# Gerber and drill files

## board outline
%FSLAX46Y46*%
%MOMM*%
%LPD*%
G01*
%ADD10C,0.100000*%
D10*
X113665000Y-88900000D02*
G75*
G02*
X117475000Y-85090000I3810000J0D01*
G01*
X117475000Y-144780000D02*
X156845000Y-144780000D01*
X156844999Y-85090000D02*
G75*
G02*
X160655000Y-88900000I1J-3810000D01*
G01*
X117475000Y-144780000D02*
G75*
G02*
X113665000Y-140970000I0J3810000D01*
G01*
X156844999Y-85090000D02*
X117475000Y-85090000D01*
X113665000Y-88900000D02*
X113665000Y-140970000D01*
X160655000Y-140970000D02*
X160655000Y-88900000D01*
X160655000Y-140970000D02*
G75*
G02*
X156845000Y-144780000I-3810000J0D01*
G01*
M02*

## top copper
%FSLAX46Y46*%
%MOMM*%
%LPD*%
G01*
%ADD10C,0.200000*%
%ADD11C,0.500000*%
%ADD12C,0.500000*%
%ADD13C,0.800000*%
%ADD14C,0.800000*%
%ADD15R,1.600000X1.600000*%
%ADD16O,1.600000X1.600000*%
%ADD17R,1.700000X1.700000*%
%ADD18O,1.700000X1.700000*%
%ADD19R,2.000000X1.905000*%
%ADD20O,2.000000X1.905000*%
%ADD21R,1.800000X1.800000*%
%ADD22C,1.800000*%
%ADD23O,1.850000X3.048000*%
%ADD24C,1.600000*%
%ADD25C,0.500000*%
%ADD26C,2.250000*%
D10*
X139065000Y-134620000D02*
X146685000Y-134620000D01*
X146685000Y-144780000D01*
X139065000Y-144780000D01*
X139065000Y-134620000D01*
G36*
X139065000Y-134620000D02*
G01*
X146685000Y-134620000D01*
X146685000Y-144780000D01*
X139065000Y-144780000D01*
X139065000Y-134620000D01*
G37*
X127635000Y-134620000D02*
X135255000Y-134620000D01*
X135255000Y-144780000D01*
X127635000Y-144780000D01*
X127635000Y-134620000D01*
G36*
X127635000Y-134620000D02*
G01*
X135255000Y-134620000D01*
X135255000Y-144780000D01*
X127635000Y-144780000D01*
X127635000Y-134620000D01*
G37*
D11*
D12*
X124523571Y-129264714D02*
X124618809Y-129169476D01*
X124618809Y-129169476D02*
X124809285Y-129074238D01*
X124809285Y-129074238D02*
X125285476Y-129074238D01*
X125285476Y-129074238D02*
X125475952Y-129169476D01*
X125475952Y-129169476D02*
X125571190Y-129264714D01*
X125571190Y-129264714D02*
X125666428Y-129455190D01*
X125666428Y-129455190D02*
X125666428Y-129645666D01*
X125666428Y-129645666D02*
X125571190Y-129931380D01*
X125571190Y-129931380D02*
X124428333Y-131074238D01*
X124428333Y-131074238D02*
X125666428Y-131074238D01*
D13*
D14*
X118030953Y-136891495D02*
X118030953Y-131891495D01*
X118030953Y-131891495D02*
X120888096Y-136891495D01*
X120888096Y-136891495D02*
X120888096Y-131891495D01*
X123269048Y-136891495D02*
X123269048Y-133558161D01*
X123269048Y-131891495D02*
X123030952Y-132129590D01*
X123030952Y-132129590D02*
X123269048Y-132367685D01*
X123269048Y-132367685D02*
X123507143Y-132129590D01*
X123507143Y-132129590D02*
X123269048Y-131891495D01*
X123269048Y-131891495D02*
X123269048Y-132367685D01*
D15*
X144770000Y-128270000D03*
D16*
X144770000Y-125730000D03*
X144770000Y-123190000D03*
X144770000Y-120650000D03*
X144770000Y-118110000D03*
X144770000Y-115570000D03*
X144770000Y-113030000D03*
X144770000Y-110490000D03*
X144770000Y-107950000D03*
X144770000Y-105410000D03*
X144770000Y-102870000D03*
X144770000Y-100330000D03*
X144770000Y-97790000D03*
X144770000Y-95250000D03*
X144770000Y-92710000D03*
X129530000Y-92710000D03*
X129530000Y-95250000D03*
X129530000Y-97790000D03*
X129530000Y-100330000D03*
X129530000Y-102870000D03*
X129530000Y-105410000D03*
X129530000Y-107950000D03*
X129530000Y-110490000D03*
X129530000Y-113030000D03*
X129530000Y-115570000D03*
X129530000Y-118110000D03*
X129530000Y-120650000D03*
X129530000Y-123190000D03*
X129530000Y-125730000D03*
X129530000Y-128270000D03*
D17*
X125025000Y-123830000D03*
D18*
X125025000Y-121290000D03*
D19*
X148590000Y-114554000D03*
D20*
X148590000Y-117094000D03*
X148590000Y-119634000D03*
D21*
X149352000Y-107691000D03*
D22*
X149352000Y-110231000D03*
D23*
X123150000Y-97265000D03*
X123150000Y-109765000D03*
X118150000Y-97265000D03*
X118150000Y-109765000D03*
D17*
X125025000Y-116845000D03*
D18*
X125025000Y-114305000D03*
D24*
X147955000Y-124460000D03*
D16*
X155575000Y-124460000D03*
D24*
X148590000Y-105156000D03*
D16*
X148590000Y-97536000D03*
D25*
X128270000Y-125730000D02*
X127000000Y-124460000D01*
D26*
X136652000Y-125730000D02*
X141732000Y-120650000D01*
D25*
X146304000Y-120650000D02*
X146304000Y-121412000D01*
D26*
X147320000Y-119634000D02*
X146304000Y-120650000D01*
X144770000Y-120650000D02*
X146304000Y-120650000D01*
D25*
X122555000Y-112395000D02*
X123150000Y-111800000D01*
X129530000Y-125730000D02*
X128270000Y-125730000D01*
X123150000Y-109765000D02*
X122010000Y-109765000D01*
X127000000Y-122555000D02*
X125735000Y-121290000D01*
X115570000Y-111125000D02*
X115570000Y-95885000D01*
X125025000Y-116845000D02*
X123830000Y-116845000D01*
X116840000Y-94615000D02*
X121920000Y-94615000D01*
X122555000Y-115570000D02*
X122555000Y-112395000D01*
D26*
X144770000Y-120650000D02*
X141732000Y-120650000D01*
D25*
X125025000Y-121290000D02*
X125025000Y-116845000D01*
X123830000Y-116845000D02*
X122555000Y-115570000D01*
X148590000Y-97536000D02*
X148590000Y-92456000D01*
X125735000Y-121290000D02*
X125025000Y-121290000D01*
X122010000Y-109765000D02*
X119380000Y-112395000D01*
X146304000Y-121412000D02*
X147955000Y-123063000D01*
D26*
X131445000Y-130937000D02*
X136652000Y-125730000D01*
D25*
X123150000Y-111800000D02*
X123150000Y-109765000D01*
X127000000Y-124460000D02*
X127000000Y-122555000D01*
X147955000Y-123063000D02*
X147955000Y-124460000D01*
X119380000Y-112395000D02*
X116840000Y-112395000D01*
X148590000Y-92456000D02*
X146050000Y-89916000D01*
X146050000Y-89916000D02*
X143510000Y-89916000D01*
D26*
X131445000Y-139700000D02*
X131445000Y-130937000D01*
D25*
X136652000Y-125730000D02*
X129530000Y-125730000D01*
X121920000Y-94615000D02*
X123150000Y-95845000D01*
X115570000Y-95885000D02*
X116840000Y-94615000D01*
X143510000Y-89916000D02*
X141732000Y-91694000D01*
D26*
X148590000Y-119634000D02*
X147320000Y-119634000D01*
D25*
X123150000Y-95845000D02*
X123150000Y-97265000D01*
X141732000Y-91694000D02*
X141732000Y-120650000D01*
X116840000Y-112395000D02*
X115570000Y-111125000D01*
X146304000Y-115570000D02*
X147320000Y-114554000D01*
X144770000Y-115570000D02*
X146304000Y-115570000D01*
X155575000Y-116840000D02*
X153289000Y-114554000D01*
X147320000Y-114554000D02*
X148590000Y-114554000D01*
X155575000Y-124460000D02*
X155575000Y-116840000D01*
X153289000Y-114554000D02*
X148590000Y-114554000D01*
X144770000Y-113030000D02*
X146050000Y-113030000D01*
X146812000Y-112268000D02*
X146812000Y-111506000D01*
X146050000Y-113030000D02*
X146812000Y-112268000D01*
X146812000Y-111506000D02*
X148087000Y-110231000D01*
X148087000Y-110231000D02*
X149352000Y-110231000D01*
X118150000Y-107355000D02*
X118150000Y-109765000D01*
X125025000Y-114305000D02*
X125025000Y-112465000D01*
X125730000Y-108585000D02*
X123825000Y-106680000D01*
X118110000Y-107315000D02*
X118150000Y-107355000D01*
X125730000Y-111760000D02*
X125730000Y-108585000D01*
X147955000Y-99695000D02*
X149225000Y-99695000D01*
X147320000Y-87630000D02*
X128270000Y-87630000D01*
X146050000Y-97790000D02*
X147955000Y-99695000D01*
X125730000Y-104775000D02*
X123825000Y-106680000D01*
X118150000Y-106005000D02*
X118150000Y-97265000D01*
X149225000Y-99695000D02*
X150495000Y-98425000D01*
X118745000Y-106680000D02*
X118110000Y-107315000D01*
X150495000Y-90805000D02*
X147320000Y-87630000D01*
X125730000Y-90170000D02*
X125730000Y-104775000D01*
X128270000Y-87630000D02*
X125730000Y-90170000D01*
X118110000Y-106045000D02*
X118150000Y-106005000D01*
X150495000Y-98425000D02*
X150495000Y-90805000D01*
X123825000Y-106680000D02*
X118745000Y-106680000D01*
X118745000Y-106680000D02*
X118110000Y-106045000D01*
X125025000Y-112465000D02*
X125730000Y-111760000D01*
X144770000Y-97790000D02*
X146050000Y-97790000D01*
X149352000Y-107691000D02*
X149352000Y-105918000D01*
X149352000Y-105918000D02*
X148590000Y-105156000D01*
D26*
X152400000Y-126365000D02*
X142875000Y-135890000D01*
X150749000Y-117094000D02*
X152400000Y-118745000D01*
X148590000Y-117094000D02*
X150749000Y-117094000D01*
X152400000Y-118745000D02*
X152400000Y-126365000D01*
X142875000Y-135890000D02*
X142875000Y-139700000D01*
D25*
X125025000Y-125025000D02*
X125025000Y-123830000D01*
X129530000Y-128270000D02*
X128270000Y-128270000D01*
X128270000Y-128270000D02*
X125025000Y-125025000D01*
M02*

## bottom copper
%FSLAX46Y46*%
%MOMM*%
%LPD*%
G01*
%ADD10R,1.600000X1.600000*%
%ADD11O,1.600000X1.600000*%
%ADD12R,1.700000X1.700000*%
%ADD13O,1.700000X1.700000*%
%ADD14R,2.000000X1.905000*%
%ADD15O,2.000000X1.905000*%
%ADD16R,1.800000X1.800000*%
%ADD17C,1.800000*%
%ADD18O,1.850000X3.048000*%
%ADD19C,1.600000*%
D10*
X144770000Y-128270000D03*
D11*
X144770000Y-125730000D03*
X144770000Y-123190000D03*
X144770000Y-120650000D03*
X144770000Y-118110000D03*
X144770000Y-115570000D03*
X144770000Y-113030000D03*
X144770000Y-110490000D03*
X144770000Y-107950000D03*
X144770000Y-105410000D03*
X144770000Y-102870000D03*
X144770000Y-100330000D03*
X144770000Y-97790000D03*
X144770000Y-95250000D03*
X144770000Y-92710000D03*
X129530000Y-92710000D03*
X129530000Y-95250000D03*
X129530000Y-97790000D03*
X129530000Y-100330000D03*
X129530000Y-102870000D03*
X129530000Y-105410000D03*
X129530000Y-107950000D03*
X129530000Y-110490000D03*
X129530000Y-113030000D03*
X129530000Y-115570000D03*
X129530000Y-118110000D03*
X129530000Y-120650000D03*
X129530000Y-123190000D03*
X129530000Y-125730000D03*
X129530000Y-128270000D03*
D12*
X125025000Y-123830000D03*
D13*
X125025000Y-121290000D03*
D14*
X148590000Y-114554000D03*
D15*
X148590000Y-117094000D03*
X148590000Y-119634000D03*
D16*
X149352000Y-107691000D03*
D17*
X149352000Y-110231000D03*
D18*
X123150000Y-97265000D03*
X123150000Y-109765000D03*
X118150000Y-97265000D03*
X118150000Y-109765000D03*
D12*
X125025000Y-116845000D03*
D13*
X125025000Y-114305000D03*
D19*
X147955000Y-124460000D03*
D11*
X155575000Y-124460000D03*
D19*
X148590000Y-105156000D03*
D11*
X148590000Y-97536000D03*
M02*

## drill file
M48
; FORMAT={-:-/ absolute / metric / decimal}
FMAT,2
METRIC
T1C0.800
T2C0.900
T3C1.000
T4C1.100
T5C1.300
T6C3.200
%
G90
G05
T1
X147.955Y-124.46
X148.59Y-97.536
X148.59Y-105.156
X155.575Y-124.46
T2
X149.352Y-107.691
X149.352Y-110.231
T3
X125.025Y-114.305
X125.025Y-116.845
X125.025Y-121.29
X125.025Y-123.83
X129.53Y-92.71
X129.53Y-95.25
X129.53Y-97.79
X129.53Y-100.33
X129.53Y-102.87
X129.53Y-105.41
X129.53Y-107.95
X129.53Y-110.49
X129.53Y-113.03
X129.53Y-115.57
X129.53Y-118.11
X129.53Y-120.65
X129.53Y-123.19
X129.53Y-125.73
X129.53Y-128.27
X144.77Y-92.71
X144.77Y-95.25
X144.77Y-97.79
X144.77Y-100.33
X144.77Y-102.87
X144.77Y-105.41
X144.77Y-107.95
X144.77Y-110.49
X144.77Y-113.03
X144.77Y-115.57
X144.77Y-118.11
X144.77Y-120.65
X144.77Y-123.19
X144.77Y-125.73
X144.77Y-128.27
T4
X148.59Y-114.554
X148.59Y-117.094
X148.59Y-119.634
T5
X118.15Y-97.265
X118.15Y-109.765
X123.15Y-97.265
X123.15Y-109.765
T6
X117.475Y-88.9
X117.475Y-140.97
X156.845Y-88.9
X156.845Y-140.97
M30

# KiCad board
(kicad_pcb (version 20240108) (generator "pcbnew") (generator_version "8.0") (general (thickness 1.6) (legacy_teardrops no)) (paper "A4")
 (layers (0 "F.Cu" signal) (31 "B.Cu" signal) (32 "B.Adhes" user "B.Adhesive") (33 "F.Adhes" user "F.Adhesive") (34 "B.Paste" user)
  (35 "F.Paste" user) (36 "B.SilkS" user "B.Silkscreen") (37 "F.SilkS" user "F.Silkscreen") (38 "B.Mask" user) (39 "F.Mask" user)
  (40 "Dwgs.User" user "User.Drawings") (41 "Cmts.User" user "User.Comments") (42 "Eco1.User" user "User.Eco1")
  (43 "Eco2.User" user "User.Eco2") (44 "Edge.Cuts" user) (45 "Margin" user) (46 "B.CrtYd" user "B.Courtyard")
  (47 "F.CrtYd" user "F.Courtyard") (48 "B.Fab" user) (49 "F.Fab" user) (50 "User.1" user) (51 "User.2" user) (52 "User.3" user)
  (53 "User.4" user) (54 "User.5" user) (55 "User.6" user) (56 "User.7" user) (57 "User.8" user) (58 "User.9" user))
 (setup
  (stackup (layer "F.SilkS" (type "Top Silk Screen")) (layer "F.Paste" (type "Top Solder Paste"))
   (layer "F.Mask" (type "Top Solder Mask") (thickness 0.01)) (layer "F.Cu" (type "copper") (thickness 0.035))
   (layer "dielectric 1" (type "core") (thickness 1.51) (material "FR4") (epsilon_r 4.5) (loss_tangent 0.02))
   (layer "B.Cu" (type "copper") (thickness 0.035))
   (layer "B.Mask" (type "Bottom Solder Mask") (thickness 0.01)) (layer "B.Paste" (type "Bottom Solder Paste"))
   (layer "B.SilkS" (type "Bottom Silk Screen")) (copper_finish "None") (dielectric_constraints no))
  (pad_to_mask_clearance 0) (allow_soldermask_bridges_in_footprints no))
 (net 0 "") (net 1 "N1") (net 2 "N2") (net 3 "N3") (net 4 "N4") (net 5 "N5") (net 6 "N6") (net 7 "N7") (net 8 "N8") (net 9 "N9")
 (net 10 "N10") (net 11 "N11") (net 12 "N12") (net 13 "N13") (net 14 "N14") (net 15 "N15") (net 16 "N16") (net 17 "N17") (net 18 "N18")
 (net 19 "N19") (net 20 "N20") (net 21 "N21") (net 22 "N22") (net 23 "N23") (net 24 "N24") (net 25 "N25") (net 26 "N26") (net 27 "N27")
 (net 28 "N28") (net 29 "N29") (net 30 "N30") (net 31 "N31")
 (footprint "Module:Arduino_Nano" (layer "F.Cu") (at 144.77 128.27 180)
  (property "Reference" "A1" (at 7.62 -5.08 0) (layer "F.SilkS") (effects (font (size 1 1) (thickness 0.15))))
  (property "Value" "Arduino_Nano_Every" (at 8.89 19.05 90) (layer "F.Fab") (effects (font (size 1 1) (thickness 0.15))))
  (pad "1" thru_hole rect (at 0 0 180) (size 1.6 1.6) (drill 1) (layers "*.Cu" "*.Mask") (remove_unused_layers no) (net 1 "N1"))
  (pad "2" thru_hole oval (at 0 2.54 180) (size 1.6 1.6) (drill 1) (layers "*.Cu" "*.Mask") (remove_unused_layers no) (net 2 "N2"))
  (pad "3" thru_hole oval (at 0 5.08 180) (size 1.6 1.6) (drill 1) (layers "*.Cu" "*.Mask") (remove_unused_layers no) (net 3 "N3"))
  (pad "4" thru_hole oval (at 0 7.62 180) (size 1.6 1.6) (drill 1) (layers "*.Cu" "*.Mask") (remove_unused_layers no) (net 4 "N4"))
  (pad "5" thru_hole oval (at 0 10.16 180) (size 1.6 1.6) (drill 1) (layers "*.Cu" "*.Mask") (remove_unused_layers no) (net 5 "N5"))
  (pad "6" thru_hole oval (at 0 12.7 180) (size 1.6 1.6) (drill 1) (layers "*.Cu" "*.Mask") (remove_unused_layers no) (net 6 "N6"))
  (pad "7" thru_hole oval (at 0 15.24 180) (size 1.6 1.6) (drill 1) (layers "*.Cu" "*.Mask") (remove_unused_layers no) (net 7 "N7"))
  (pad "8" thru_hole oval (at 0 17.78 180) (size 1.6 1.6) (drill 1) (layers "*.Cu" "*.Mask") (remove_unused_layers no) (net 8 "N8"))
  (pad "9" thru_hole oval (at 0 20.32 180) (size 1.6 1.6) (drill 1) (layers "*.Cu" "*.Mask") (remove_unused_layers no) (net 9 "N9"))
  (pad "10" thru_hole oval (at 0 22.86 180) (size 1.6 1.6) (drill 1) (layers "*.Cu" "*.Mask") (remove_unused_layers no) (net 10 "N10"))
  (pad "11" thru_hole oval (at 0 25.4 180) (size 1.6 1.6) (drill 1) (layers "*.Cu" "*.Mask") (remove_unused_layers no) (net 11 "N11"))
  (pad "12" thru_hole oval (at 0 27.94 180) (size 1.6 1.6) (drill 1) (layers "*.Cu" "*.Mask") (remove_unused_layers no) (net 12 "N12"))
  (pad "13" thru_hole oval (at 0 30.48 180) (size 1.6 1.6) (drill 1) (layers "*.Cu" "*.Mask") (remove_unused_layers no) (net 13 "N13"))
  (pad "14" thru_hole oval (at 0 33.02 180) (size 1.6 1.6) (drill 1) (layers "*.Cu" "*.Mask") (remove_unused_layers no) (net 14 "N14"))
  (pad "15" thru_hole oval (at 0 35.56 180) (size 1.6 1.6) (drill 1) (layers "*.Cu" "*.Mask") (remove_unused_layers no) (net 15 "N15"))
  (pad "16" thru_hole oval (at 15.24 35.56 180) (size 1.6 1.6) (drill 1) (layers "*.Cu" "*.Mask") (remove_unused_layers no) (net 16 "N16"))
  (pad "17" thru_hole oval (at 15.24 33.02 180) (size 1.6 1.6) (drill 1) (layers "*.Cu" "*.Mask") (remove_unused_layers no) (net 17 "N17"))
  (pad "18" thru_hole oval (at 15.24 30.48 180) (size 1.6 1.6) (drill 1) (layers "*.Cu" "*.Mask") (remove_unused_layers no) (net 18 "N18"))
  (pad "19" thru_hole oval (at 15.24 27.94 180) (size 1.6 1.6) (drill 1) (layers "*.Cu" "*.Mask") (remove_unused_layers no) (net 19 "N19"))
  (pad "20" thru_hole oval (at 15.24 25.4 180) (size 1.6 1.6) (drill 1) (layers "*.Cu" "*.Mask") (remove_unused_layers no) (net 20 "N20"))
  (pad "21" thru_hole oval (at 15.24 22.86 180) (size 1.6 1.6) (drill 1) (layers "*.Cu" "*.Mask") (remove_unused_layers no) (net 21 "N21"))
  (pad "22" thru_hole oval (at 15.24 20.32 180) (size 1.6 1.6) (drill 1) (layers "*.Cu" "*.Mask") (remove_unused_layers no) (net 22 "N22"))
  (pad "23" thru_hole oval (at 15.24 17.78 180) (size 1.6 1.6) (drill 1) (layers "*.Cu" "*.Mask") (remove_unused_layers no) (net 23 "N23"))
  (pad "24" thru_hole oval (at 15.24 15.24 180) (size 1.6 1.6) (drill 1) (layers "*.Cu" "*.Mask") (remove_unused_layers no) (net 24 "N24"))
  (pad "25" thru_hole oval (at 15.24 12.7 180) (size 1.6 1.6) (drill 1) (layers "*.Cu" "*.Mask") (remove_unused_layers no) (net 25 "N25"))
  (pad "26" thru_hole oval (at 15.24 10.16 180) (size 1.6 1.6) (drill 1) (layers "*.Cu" "*.Mask") (remove_unused_layers no) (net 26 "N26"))
  (pad "27" thru_hole oval (at 15.24 7.62 180) (size 1.6 1.6) (drill 1) (layers "*.Cu" "*.Mask") (remove_unused_layers no) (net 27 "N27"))
  (pad "28" thru_hole oval (at 15.24 5.08 180) (size 1.6 1.6) (drill 1) (layers "*.Cu" "*.Mask") (remove_unused_layers no) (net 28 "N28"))
  (pad "29" thru_hole oval (at 15.24 2.54 180) (size 1.6 1.6) (drill 1) (layers "*.Cu" "*.Mask") (remove_unused_layers no) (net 4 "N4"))
  (pad "30" thru_hole oval (at 15.24 0 180) (size 1.6 1.6) (drill 1) (layers "*.Cu" "*.Mask") (remove_unused_layers no) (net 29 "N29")))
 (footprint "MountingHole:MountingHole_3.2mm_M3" (layer "F.Cu") (at 156.845 140.97)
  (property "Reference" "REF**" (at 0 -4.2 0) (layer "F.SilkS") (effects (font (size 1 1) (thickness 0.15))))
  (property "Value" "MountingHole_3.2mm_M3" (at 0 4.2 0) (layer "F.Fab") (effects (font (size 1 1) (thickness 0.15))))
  (pad "" np_thru_hole circle (at 0 0) (size 3.2 3.2) (drill 3.2) (layers "F&B.Cu" "*.Mask")))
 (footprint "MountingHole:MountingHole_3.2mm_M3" (layer "F.Cu") (at 156.845 88.9)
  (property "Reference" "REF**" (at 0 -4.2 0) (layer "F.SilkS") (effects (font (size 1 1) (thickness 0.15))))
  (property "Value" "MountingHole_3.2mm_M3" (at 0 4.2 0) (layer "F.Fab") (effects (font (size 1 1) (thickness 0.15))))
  (pad "" np_thru_hole circle (at 0 0) (size 3.2 3.2) (drill 3.2) (layers "F&B.Cu" "*.Mask")))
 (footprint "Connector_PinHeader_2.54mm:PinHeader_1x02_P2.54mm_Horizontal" (layer "F.Cu") (at 125.025 123.83 180)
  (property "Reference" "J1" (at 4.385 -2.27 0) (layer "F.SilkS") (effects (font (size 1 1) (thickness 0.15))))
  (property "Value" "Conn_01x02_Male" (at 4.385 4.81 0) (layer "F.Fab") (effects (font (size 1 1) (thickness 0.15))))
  (pad "1" thru_hole rect (at 0 0 180) (size 1.7 1.7) (drill 1) (layers "*.Cu" "*.Mask") (remove_unused_layers no) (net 29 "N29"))
  (pad "2" thru_hole oval (at 0 2.54 180) (size 1.7 1.7) (drill 1) (layers "*.Cu" "*.Mask") (remove_unused_layers no) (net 4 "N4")))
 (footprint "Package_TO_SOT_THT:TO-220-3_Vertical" (layer "F.Cu") (at 148.59 114.554 -90)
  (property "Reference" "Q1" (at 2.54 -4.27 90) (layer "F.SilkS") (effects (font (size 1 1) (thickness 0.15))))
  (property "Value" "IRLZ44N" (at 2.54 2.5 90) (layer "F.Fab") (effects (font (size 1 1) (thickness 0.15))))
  (pad "1" thru_hole rect (at 0 0 270) (size 1.905 2) (drill 1.1) (layers "*.Cu" "*.Mask") (remove_unused_layers no) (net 6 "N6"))
  (pad "2" thru_hole oval (at 2.54 0 270) (size 1.905 2) (drill 1.1) (layers "*.Cu" "*.Mask") (remove_unused_layers no) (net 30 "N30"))
  (pad "3" thru_hole oval (at 5.08 0 270) (size 1.905 2) (drill 1.1) (layers "*.Cu" "*.Mask") (remove_unused_layers no) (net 4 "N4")))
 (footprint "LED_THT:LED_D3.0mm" (layer "F.Cu") (at 149.352 107.691 -90)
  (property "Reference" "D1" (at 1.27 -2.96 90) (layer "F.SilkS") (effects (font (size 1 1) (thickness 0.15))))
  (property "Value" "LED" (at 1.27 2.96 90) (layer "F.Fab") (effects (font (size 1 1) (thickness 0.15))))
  (pad "1" thru_hole rect (at 0 0 270) (size 1.8 1.8) (drill 0.9) (layers "*.Cu" "*.Mask") (remove_unused_layers no) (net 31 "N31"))
  (pad "2" thru_hole circle (at 2.54 0 270) (size 1.8 1.8) (drill 0.9) (layers "*.Cu" "*.Mask") (remove_unused_layers no) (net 7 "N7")))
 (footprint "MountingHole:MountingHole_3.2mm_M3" (layer "F.Cu") (at 117.475 140.97)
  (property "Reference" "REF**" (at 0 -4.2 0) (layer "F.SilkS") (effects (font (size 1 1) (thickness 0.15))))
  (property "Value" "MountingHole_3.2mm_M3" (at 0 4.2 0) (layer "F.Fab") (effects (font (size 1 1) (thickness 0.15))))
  (pad "" np_thru_hole circle (at 0 0) (size 3.2 3.2) (drill 3.2) (layers "*.Cu" "*.Mask")))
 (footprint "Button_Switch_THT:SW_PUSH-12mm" (layer "F.Cu") (at 123.15 97.265 -90)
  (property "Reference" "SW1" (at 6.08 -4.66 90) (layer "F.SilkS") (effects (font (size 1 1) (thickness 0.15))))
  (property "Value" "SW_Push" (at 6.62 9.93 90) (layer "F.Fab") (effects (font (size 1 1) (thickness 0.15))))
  (pad "1" thru_hole oval (at 0 0 270) (size 3.048 1.85) (drill 1.3) (layers "*.Cu" "*.Mask") (remove_unused_layers no) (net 4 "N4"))
  (pad "1" thru_hole oval (at 12.5 0 270) (size 3.048 1.85) (drill 1.3) (layers "*.Cu" "*.Mask") (remove_unused_layers no) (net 4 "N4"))
  (pad "2" thru_hole oval (at 0 5 270) (size 3.048 1.85) (drill 1.3) (layers "*.Cu" "*.Mask") (remove_unused_layers no) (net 13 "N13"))
  (pad "2" thru_hole oval (at 12.5 5 270) (size 3.048 1.85) (drill 1.3) (layers "*.Cu" "*.Mask") (remove_unused_layers no) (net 13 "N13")))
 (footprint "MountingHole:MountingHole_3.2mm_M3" (layer "F.Cu") (at 117.475 88.9)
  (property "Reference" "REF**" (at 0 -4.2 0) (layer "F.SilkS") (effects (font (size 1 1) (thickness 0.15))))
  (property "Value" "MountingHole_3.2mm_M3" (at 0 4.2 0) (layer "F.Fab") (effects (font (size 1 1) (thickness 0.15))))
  (pad "" np_thru_hole circle (at 0 0) (size 3.2 3.2) (drill 3.2) (layers "F&B.Cu" "*.Mask")))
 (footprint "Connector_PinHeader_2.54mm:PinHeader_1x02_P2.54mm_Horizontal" (layer "F.Cu") (at 125.025 116.845 180)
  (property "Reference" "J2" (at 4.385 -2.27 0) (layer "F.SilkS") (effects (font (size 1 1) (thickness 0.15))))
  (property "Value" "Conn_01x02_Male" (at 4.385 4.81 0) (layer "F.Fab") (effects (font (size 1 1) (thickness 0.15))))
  (pad "1" thru_hole rect (at 0 0 180) (size 1.7 1.7) (drill 1) (layers "*.Cu" "*.Mask") (remove_unused_layers no) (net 4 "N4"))
  (pad "2" thru_hole oval (at 0 2.54 180) (size 1.7 1.7) (drill 1) (layers "*.Cu" "*.Mask") (remove_unused_layers no) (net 13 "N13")))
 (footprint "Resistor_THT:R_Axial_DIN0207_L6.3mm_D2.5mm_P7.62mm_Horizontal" (layer "F.Cu") (at 147.955 124.46)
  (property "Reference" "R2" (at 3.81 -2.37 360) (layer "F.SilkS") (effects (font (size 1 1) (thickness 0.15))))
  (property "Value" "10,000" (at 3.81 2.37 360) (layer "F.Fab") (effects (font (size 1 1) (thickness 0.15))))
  (pad "1" thru_hole circle (at 0 0) (size 1.6 1.6) (drill 0.8) (layers "*.Cu" "*.Mask") (remove_unused_layers no) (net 4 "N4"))
  (pad "2" thru_hole oval (at 7.62 0) (size 1.6 1.6) (drill 0.8) (layers "*.Cu" "*.Mask") (remove_unused_layers no) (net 6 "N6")))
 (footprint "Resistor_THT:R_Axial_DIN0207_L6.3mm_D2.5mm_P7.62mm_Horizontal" (layer "F.Cu") (at 148.59 105.156 90)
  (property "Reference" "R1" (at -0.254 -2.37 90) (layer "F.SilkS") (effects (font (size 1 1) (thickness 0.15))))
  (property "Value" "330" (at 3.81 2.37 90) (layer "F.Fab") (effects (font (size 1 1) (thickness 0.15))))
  (pad "1" thru_hole circle (at 0 0 90) (size 1.6 1.6) (drill 0.8) (layers "*.Cu" "*.Mask") (remove_unused_layers no) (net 31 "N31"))
  (pad "2" thru_hole oval (at 7.62 0 90) (size 1.6 1.6) (drill 0.8) (layers "*.Cu" "*.Mask") (remove_unused_layers no) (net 4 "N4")))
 (gr_rect (start 139.065 134.62) (end 146.685 144.78) (stroke (width 0.2) (type solid)) (fill solid) (layer "F.Cu") (net 30))
 (gr_rect (start 127.635 134.62) (end 135.255 144.78) (stroke (width 0.2) (type solid)) (fill solid) (layer "F.Cu") (net 4))
 (gr_arc (start 113.665 88.9) (mid 114.780923 86.205923) (end 117.475 85.09) (stroke (width 0.1) (type default)) (layer "Edge.Cuts"))
 (gr_line (start 117.475 144.78) (end 156.845 144.78) (stroke (width 0.1) (type solid)) (layer "Edge.Cuts"))
 (gr_arc (start 156.844999 85.09) (mid 159.539076 86.205923) (end 160.654999 88.9) (stroke (width 0.1) (type solid)) (layer "Edge.Cuts"))
 (gr_arc (start 117.475 144.78) (mid 114.780923 143.664077) (end 113.665 140.97) (stroke (width 0.1) (type solid)) (layer "Edge.Cuts"))
 (gr_line (start 156.844999 85.09) (end 117.475 85.09) (stroke (width 0.1) (type solid)) (layer "Edge.Cuts"))
 (gr_line (start 113.665 88.9) (end 113.665 140.97) (stroke (width 0.1) (type solid)) (layer "Edge.Cuts"))
 (gr_line (start 160.655 140.97) (end 160.655 88.9) (stroke (width 0.1) (type solid)) (layer "Edge.Cuts"))
 (gr_arc (start 160.655 140.97) (mid 159.539077 143.664077) (end 156.845 144.78) (stroke (width 0.1) (type solid)) (layer "Edge.Cuts"))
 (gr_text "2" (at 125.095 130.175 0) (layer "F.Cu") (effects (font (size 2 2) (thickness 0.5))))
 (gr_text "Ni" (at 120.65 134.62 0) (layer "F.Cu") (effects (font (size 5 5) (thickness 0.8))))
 (segment (start 128.27 125.73) (end 127 124.46) (width 0.5) (layer "F.Cu") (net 4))
 (segment (start 136.652 125.73) (end 141.732 120.65) (width 2.25) (layer "F.Cu") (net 4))
 (segment (start 146.304 120.65) (end 146.304 121.412) (width 0.5) (layer "F.Cu") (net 4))
 (segment (start 147.32 119.634) (end 146.304 120.65) (width 2.25) (layer "F.Cu") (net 4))
 (segment (start 144.77 120.65) (end 146.304 120.65) (width 2.25) (layer "F.Cu") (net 4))
 (segment (start 122.555 112.395) (end 123.15 111.8) (width 0.5) (layer "F.Cu") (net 4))
 (segment (start 129.53 125.73) (end 128.27 125.73) (width 0.5) (layer "F.Cu") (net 4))
 (segment (start 123.15 109.765) (end 122.01 109.765) (width 0.5) (layer "F.Cu") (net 4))
 (segment (start 127 122.555) (end 125.735 121.29) (width 0.5) (layer "F.Cu") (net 4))
 (segment (start 115.57 111.125) (end 115.57 95.885) (width 0.5) (layer "F.Cu") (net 4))
 (segment (start 125.025 116.845) (end 123.83 116.845) (width 0.5) (layer "F.Cu") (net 4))
 (segment (start 116.84 94.615) (end 121.92 94.615) (width 0.5) (layer "F.Cu") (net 4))
 (segment (start 122.555 115.57) (end 122.555 112.395) (width 0.5) (layer "F.Cu") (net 4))
 (segment (start 144.77 120.65) (end 141.732 120.65) (width 2.25) (layer "F.Cu") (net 4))
 (segment (start 125.025 121.29) (end 125.025 116.845) (width 0.5) (layer "F.Cu") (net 4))
 (segment (start 123.83 116.845) (end 122.555 115.57) (width 0.5) (layer "F.Cu") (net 4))
 (segment (start 148.59 97.536) (end 148.59 92.456) (width 0.5) (layer "F.Cu") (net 4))
 (segment (start 125.735 121.29) (end 125.025 121.29) (width 0.5) (layer "F.Cu") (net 4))
 (segment (start 122.01 109.765) (end 119.38 112.395) (width 0.5) (layer "F.Cu") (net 4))
 (segment (start 146.304 121.412) (end 147.955 123.063) (width 0.5) (layer "F.Cu") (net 4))
 (segment (start 131.445 130.937) (end 136.652 125.73) (width 2.25) (layer "F.Cu") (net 4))
 (segment (start 123.15 111.8) (end 123.15 109.765) (width 0.5) (layer "F.Cu") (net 4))
 (segment (start 127 124.46) (end 127 122.555) (width 0.5) (layer "F.Cu") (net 4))
 (segment (start 147.955 123.063) (end 147.955 124.46) (width 0.5) (layer "F.Cu") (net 4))
 (segment (start 119.38 112.395) (end 116.84 112.395) (width 0.5) (layer "F.Cu") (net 4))
 (segment (start 148.59 92.456) (end 146.05 89.916) (width 0.5) (layer "F.Cu") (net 4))
 (segment (start 146.05 89.916) (end 143.51 89.916) (width 0.5) (layer "F.Cu") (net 4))
 (segment (start 131.445 139.7) (end 131.445 130.937) (width 2.25) (layer "F.Cu") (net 4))
 (segment (start 136.652 125.73) (end 129.53 125.73) (width 0.5) (layer "F.Cu") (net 4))
 (segment (start 121.92 94.615) (end 123.15 95.845) (width 0.5) (layer "F.Cu") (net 4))
 (segment (start 115.57 95.885) (end 116.84 94.615) (width 0.5) (layer "F.Cu") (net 4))
 (segment (start 143.51 89.916) (end 141.732 91.694) (width 0.5) (layer "F.Cu") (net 4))
 (segment (start 148.59 119.634) (end 147.32 119.634) (width 2.25) (layer "F.Cu") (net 4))
 (segment (start 123.15 95.845) (end 123.15 97.265) (width 0.5) (layer "F.Cu") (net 4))
 (segment (start 141.732 91.694) (end 141.732 120.65) (width 0.5) (layer "F.Cu") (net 4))
 (segment (start 116.84 112.395) (end 115.57 111.125) (width 0.5) (layer "F.Cu") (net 4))
 (segment (start 146.304 115.57) (end 147.32 114.554) (width 0.5) (layer "F.Cu") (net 6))
 (segment (start 144.77 115.57) (end 146.304 115.57) (width 0.5) (layer "F.Cu") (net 6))
 (segment (start 155.575 116.84) (end 153.289 114.554) (width 0.5) (layer "F.Cu") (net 6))
 (segment (start 147.32 114.554) (end 148.59 114.554) (width 0.5) (layer "F.Cu") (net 6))
 (segment (start 155.575 124.46) (end 155.575 116.84) (width 0.5) (layer "F.Cu") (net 6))
 (segment (start 153.289 114.554) (end 148.59 114.554) (width 0.5) (layer "F.Cu") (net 6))
 (segment (start 144.77 113.03) (end 146.05 113.03) (width 0.5) (layer "F.Cu") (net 7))
 (segment (start 146.812 112.268) (end 146.812 111.506) (width 0.5) (layer "F.Cu") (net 7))
 (segment (start 146.05 113.03) (end 146.812 112.268) (width 0.5) (layer "F.Cu") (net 7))
 (segment (start 146.812 111.506) (end 148.087 110.231) (width 0.5) (layer "F.Cu") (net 7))
 (segment (start 148.087 110.231) (end 149.352 110.231) (width 0.5) (layer "F.Cu") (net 7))
 (segment (start 118.15 107.355) (end 118.15 109.765) (width 0.5) (layer "F.Cu") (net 13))
 (segment (start 125.025 114.305) (end 125.025 112.465) (width 0.5) (layer "F.Cu") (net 13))
 (segment (start 125.73 108.585) (end 123.825 106.68) (width 0.5) (layer "F.Cu") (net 13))
 (segment (start 118.11 107.315) (end 118.15 107.355) (width 0.5) (layer "F.Cu") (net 13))
 (segment (start 125.73 111.76) (end 125.73 108.585) (width 0.5) (layer "F.Cu") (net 13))
 (segment (start 147.955 99.695) (end 149.225 99.695) (width 0.5) (layer "F.Cu") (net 13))
 (segment (start 147.32 87.63) (end 128.27 87.63) (width 0.5) (layer "F.Cu") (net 13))
 (segment (start 146.05 97.79) (end 147.955 99.695) (width 0.5) (layer "F.Cu") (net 13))
 (segment (start 125.73 104.775) (end 123.825 106.68) (width 0.5) (layer "F.Cu") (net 13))
 (segment (start 118.15 106.005) (end 118.15 97.265) (width 0.5) (layer "F.Cu") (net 13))
 (segment (start 149.225 99.695) (end 150.495 98.425) (width 0.5) (layer "F.Cu") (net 13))
 (segment (start 118.745 106.68) (end 118.11 107.315) (width 0.5) (layer "F.Cu") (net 13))
 (segment (start 150.495 90.805) (end 147.32 87.63) (width 0.5) (layer "F.Cu") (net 13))
 (segment (start 125.73 90.17) (end 125.73 104.775) (width 0.5) (layer "F.Cu") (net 13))
 (segment (start 128.27 87.63) (end 125.73 90.17) (width 0.5) (layer "F.Cu") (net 13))
 (segment (start 118.11 106.045) (end 118.15 106.005) (width 0.5) (layer "F.Cu") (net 13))
 (segment (start 150.495 98.425) (end 150.495 90.805) (width 0.5) (layer "F.Cu") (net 13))
 (segment (start 123.825 106.68) (end 118.745 106.68) (width 0.5) (layer "F.Cu") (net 13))
 (segment (start 118.745 106.68) (end 118.11 106.045) (width 0.5) (layer "F.Cu") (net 13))
 (segment (start 125.025 112.465) (end 125.73 111.76) (width 0.5) (layer "F.Cu") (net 13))
 (segment (start 144.77 97.79) (end 146.05 97.79) (width 0.5) (layer "F.Cu") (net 13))
 (segment (start 149.352 107.691) (end 149.352 105.918) (width 0.5) (layer "F.Cu") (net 31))
 (segment (start 149.352 105.918) (end 148.59 105.156) (width 0.5) (layer "F.Cu") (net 31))
 (segment (start 152.4 126.365) (end 142.875 135.89) (width 2.25) (layer "F.Cu") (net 30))
 (segment (start 150.749 117.094) (end 152.4 118.745) (width 2.25) (layer "F.Cu") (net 30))
 (segment (start 148.59 117.094) (end 150.749 117.094) (width 2.25) (layer "F.Cu") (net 30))
 (segment (start 152.4 118.745) (end 152.4 126.365) (width 2.25) (layer "F.Cu") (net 30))
 (segment (start 142.875 135.89) (end 142.875 139.7) (width 2.25) (layer "F.Cu") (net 30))
 (segment (start 125.025 125.025) (end 125.025 123.83) (width 0.5) (layer "F.Cu") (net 29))
 (segment (start 129.53 128.27) (end 128.27 128.27) (width 0.5) (layer "F.Cu") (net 29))
 (segment (start 128.27 128.27) (end 125.025 125.025) (width 0.5) (layer "F.Cu") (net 29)))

